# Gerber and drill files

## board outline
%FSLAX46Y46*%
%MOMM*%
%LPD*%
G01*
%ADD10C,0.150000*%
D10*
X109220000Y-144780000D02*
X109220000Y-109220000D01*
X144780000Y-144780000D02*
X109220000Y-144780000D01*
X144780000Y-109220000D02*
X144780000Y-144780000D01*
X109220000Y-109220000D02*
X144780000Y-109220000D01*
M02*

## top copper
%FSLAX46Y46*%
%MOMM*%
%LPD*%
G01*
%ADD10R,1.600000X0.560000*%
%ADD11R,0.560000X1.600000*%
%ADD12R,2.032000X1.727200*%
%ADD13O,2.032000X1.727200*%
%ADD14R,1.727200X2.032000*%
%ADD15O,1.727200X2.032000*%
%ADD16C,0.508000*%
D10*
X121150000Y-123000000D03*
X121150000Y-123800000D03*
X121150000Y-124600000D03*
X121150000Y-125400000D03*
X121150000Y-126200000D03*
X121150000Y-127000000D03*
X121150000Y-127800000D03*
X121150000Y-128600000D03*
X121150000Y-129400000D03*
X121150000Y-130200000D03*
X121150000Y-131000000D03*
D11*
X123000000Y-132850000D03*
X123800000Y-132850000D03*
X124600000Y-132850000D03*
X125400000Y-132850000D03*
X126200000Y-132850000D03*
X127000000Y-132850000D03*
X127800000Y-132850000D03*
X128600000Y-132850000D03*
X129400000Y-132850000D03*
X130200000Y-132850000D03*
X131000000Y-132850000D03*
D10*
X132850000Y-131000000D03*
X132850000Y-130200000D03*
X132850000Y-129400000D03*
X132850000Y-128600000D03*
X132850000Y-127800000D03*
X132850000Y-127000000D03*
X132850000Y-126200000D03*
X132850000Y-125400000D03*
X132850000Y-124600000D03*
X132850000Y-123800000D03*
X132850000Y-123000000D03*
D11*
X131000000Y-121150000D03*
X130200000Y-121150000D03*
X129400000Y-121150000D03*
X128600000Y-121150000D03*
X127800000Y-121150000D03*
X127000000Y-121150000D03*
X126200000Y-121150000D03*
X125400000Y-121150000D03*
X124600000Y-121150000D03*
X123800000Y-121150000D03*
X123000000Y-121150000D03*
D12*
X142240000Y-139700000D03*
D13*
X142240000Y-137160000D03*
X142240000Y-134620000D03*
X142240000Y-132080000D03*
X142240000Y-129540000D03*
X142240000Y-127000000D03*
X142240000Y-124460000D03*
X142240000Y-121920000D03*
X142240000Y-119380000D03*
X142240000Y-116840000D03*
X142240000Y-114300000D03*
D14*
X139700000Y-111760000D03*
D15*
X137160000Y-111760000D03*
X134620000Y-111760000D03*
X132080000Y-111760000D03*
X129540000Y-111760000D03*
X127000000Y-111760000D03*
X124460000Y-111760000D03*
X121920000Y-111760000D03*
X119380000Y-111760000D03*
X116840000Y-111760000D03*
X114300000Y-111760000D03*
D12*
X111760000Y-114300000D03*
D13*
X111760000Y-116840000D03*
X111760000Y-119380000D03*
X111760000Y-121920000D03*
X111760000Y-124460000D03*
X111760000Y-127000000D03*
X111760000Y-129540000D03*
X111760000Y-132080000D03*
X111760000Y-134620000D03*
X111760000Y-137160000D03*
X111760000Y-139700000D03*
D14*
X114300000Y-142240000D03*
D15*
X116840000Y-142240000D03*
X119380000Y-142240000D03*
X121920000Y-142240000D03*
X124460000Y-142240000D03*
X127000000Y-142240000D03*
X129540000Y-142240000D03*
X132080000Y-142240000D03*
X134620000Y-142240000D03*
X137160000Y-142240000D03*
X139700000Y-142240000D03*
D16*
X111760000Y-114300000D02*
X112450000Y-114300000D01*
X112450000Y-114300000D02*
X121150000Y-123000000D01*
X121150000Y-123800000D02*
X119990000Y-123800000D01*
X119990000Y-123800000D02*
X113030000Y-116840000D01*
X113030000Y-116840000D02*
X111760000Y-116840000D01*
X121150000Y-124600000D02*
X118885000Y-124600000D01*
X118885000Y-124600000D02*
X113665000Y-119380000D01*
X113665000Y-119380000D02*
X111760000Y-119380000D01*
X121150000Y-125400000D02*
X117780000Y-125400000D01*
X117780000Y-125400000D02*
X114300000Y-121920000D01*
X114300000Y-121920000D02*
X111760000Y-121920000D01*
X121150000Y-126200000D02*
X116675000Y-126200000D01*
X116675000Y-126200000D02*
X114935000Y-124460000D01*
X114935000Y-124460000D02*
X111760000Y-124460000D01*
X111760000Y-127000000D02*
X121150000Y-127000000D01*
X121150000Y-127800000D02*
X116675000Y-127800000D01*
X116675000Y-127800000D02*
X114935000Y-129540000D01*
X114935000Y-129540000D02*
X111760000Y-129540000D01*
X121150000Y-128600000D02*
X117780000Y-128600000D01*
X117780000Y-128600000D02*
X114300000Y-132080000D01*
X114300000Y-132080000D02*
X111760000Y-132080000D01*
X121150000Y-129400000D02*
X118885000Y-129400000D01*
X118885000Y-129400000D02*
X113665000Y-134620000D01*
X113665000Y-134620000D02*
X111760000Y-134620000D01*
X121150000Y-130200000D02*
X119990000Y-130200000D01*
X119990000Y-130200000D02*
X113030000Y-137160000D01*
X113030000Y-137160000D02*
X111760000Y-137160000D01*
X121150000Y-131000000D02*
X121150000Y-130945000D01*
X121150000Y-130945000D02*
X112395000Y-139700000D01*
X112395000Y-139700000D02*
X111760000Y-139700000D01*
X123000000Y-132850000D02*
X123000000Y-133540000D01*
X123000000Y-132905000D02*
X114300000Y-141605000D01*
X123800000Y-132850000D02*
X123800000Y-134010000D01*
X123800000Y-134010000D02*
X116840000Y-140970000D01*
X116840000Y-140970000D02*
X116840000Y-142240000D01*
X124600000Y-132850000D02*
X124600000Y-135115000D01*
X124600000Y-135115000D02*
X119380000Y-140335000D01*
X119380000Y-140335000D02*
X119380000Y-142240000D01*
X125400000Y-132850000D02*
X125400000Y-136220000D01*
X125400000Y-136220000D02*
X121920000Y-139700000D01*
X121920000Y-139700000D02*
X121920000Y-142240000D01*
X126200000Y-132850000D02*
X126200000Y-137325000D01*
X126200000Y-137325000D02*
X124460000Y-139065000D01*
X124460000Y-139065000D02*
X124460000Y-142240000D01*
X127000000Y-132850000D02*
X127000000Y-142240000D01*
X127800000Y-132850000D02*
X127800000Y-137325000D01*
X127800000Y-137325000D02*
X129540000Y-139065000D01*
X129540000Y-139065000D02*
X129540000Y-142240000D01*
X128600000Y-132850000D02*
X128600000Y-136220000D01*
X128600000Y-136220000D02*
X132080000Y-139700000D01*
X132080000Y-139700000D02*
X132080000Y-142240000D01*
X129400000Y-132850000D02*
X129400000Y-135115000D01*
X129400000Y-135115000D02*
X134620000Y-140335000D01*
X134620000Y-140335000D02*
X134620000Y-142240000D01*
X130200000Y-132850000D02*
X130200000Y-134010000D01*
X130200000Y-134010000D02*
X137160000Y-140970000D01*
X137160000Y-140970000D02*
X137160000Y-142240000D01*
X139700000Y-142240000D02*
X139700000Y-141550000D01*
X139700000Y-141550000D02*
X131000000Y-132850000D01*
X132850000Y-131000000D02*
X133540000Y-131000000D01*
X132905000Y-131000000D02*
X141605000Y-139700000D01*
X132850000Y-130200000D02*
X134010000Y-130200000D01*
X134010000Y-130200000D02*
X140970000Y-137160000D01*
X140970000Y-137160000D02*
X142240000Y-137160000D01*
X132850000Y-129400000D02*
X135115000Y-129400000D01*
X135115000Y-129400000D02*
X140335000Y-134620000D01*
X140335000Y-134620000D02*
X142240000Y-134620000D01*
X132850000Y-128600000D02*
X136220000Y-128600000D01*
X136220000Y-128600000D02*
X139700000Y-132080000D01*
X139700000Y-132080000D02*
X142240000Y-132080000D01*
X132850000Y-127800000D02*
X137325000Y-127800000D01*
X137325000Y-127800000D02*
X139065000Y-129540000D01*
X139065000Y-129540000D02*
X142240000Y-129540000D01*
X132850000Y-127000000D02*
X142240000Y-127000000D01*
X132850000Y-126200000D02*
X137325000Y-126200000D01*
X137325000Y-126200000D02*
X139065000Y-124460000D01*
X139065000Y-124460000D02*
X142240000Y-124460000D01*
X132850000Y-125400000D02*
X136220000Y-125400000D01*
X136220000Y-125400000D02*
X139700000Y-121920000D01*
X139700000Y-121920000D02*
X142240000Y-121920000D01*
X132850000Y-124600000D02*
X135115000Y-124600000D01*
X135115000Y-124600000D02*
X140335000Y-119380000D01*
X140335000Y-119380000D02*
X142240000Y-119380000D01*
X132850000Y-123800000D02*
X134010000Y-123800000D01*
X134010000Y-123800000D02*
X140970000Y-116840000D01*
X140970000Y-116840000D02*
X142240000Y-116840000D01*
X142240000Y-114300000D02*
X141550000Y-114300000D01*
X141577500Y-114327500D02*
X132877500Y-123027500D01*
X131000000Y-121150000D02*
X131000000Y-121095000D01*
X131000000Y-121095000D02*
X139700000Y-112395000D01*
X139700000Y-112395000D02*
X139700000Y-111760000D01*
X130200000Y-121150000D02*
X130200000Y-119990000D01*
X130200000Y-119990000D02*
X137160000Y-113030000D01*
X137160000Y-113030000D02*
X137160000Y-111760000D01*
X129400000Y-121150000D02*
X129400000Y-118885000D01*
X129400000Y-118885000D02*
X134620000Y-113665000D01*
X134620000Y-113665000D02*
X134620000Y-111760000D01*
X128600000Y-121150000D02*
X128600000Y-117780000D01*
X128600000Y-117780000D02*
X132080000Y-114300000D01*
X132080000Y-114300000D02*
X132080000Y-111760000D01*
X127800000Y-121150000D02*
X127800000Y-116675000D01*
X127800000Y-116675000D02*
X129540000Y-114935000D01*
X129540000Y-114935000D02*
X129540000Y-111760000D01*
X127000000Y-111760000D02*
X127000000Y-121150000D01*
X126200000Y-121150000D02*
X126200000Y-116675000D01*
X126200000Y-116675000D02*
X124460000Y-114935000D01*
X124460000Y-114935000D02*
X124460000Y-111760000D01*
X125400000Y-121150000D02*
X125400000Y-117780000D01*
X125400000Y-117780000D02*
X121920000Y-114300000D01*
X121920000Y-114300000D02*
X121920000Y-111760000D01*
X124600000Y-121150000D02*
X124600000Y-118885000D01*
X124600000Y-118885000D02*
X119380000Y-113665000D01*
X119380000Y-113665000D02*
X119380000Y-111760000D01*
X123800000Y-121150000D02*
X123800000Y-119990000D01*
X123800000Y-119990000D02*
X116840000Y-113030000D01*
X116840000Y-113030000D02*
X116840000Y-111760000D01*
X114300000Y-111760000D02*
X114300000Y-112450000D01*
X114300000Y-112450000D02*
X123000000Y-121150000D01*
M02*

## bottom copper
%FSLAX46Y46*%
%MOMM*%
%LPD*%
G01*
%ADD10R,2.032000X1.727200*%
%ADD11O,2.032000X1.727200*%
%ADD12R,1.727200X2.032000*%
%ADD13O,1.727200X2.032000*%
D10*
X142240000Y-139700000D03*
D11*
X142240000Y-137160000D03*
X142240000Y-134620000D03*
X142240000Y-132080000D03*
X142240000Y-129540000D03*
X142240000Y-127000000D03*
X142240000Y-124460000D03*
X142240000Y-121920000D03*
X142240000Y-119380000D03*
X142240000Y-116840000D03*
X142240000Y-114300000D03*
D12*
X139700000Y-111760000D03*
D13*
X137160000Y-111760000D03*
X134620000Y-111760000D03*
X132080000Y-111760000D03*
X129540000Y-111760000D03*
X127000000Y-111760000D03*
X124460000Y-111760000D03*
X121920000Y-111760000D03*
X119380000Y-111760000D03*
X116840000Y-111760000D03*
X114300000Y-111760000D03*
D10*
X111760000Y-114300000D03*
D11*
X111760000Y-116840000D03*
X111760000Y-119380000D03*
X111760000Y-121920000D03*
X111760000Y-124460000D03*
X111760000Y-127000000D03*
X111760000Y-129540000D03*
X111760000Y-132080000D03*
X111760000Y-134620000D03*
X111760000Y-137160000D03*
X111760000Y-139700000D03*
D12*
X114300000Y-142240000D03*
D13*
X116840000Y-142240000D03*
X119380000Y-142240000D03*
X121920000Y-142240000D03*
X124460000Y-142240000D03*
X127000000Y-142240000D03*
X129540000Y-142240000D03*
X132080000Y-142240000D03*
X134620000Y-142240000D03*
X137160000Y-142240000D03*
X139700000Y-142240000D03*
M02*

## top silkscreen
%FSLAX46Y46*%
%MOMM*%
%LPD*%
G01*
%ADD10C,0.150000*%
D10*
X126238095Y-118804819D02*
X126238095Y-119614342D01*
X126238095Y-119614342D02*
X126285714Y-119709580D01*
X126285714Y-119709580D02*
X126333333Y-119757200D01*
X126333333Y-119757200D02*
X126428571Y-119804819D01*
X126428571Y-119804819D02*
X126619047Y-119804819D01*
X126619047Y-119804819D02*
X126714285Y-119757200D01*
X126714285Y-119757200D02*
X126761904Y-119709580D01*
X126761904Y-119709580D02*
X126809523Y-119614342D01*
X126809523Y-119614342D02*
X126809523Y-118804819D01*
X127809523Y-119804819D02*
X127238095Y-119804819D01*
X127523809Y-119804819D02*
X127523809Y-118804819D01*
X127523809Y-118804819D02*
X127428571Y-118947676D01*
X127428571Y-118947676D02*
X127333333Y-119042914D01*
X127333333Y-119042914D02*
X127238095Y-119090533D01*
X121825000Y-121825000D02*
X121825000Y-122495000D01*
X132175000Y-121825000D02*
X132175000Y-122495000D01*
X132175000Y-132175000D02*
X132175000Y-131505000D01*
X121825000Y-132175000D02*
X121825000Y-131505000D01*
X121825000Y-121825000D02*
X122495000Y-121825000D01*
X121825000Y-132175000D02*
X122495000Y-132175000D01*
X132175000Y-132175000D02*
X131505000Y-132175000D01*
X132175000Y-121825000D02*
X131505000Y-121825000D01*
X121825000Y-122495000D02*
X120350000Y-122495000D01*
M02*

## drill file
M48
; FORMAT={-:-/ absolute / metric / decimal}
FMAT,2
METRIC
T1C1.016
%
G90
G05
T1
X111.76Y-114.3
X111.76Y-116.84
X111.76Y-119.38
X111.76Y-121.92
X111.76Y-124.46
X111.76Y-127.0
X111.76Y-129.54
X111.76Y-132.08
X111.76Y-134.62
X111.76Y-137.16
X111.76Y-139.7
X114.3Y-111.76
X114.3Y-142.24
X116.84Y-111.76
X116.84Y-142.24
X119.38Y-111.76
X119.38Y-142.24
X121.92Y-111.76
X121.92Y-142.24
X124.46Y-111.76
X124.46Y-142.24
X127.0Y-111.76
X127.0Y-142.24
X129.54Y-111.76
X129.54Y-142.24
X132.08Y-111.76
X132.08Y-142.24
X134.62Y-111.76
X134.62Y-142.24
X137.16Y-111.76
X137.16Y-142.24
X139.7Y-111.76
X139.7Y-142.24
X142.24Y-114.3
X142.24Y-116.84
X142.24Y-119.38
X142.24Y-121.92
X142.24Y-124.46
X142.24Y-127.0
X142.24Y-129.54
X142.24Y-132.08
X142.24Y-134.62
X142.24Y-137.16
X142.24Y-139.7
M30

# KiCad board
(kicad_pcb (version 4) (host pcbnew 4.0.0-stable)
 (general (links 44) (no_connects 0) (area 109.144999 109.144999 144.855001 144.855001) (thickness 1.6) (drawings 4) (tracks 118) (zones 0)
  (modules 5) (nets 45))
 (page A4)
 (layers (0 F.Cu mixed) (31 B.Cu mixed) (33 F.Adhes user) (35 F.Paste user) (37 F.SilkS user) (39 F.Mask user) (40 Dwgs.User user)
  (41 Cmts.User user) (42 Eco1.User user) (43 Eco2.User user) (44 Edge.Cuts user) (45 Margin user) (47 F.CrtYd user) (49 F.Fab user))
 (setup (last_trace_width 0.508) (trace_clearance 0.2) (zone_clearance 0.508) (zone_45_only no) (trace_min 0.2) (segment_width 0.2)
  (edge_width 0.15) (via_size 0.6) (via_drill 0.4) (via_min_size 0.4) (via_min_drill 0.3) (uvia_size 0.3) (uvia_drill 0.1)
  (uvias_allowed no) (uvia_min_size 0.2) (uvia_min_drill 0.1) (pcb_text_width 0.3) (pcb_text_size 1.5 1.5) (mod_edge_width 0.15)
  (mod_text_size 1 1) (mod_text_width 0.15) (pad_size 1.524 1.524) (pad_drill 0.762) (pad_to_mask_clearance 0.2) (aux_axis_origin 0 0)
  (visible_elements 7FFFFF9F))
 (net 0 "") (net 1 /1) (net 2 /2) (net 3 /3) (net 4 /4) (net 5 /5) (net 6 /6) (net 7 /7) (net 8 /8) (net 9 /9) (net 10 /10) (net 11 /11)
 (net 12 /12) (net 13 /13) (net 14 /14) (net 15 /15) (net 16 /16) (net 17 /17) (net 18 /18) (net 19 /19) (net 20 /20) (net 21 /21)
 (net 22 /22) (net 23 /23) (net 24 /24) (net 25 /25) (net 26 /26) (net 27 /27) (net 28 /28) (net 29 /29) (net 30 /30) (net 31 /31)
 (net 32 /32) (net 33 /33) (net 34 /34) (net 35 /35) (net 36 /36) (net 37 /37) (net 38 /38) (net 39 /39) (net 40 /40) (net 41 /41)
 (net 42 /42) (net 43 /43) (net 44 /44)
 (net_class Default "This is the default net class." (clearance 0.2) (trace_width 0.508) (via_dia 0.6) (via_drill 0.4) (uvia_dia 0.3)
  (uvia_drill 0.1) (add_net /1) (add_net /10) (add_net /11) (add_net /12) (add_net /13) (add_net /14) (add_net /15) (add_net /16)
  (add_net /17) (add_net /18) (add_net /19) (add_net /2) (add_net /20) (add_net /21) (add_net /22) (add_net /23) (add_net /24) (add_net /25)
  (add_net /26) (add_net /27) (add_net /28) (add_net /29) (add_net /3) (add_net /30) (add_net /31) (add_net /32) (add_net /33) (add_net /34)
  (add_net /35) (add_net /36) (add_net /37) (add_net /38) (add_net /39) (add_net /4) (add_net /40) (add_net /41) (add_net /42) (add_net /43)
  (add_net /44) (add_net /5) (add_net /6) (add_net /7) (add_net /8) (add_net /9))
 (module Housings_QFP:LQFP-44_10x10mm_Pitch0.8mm (layer F.Cu) (at 127 127)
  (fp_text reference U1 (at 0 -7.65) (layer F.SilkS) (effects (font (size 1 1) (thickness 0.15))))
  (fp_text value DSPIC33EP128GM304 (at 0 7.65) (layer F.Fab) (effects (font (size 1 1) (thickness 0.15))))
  (fp_line (start -5.175 -5.175) (end -5.175 -4.505) (layer F.SilkS) (width 0.15))
  (fp_line (start 5.175 -5.175) (end 5.175 -4.505) (layer F.SilkS) (width 0.15))
  (fp_line (start 5.175 5.175) (end 5.175 4.505) (layer F.SilkS) (width 0.15))
  (fp_line (start -5.175 5.175) (end -5.175 4.505) (layer F.SilkS) (width 0.15))
  (fp_line (start -5.175 -5.175) (end -4.505 -5.175) (layer F.SilkS) (width 0.15))
  (fp_line (start -5.175 5.175) (end -4.505 5.175) (layer F.SilkS) (width 0.15))
  (fp_line (start 5.175 5.175) (end 4.505 5.175) (layer F.SilkS) (width 0.15))
  (fp_line (start 5.175 -5.175) (end 4.505 -5.175) (layer F.SilkS) (width 0.15))
  (fp_line (start -5.175 -4.505) (end -6.65 -4.505) (layer F.SilkS) (width 0.15))
  (pad 1 smd rect (at -5.85 -4) (size 1.6 0.56) (layers F.Cu F.Paste F.Mask) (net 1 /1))
  (pad 2 smd rect (at -5.85 -3.2) (size 1.6 0.56) (layers F.Cu F.Paste F.Mask) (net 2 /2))
  (pad 3 smd rect (at -5.85 -2.4) (size 1.6 0.56) (layers F.Cu F.Paste F.Mask) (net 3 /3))
  (pad 4 smd rect (at -5.85 -1.6) (size 1.6 0.56) (layers F.Cu F.Paste F.Mask) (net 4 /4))
  (pad 5 smd rect (at -5.85 -0.8) (size 1.6 0.56) (layers F.Cu F.Paste F.Mask) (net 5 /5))
  (pad 6 smd rect (at -5.85 0) (size 1.6 0.56) (layers F.Cu F.Paste F.Mask) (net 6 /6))
  (pad 7 smd rect (at -5.85 0.8) (size 1.6 0.56) (layers F.Cu F.Paste F.Mask) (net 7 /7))
  (pad 8 smd rect (at -5.85 1.6) (size 1.6 0.56) (layers F.Cu F.Paste F.Mask) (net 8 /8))
  (pad 9 smd rect (at -5.85 2.4) (size 1.6 0.56) (layers F.Cu F.Paste F.Mask) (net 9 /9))
  (pad 10 smd rect (at -5.85 3.2) (size 1.6 0.56) (layers F.Cu F.Paste F.Mask) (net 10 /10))
  (pad 11 smd rect (at -5.85 4) (size 1.6 0.56) (layers F.Cu F.Paste F.Mask) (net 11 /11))
  (pad 12 smd rect (at -4 5.85 90) (size 1.6 0.56) (layers F.Cu F.Paste F.Mask) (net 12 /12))
  (pad 13 smd rect (at -3.2 5.85 90) (size 1.6 0.56) (layers F.Cu F.Paste F.Mask) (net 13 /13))
  (pad 14 smd rect (at -2.4 5.85 90) (size 1.6 0.56) (layers F.Cu F.Paste F.Mask) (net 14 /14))
  (pad 15 smd rect (at -1.6 5.85 90) (size 1.6 0.56) (layers F.Cu F.Paste F.Mask) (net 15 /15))
  (pad 16 smd rect (at -0.8 5.85 90) (size 1.6 0.56) (layers F.Cu F.Paste F.Mask) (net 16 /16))
  (pad 17 smd rect (at 0 5.85 90) (size 1.6 0.56) (layers F.Cu F.Paste F.Mask) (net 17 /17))
  (pad 18 smd rect (at 0.8 5.85 90) (size 1.6 0.56) (layers F.Cu F.Paste F.Mask) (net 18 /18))
  (pad 19 smd rect (at 1.6 5.85 90) (size 1.6 0.56) (layers F.Cu F.Paste F.Mask) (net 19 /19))
  (pad 20 smd rect (at 2.4 5.85 90) (size 1.6 0.56) (layers F.Cu F.Paste F.Mask) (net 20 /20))
  (pad 21 smd rect (at 3.2 5.85 90) (size 1.6 0.56) (layers F.Cu F.Paste F.Mask) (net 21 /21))
  (pad 22 smd rect (at 4 5.85 90) (size 1.6 0.56) (layers F.Cu F.Paste F.Mask) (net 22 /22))
  (pad 23 smd rect (at 5.85 4) (size 1.6 0.56) (layers F.Cu F.Paste F.Mask) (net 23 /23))
  (pad 24 smd rect (at 5.85 3.2) (size 1.6 0.56) (layers F.Cu F.Paste F.Mask) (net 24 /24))
  (pad 25 smd rect (at 5.85 2.4) (size 1.6 0.56) (layers F.Cu F.Paste F.Mask) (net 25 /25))
  (pad 26 smd rect (at 5.85 1.6) (size 1.6 0.56) (layers F.Cu F.Paste F.Mask) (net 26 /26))
  (pad 27 smd rect (at 5.85 0.8) (size 1.6 0.56) (layers F.Cu F.Paste F.Mask) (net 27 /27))
  (pad 28 smd rect (at 5.85 0) (size 1.6 0.56) (layers F.Cu F.Paste F.Mask) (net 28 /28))
  (pad 29 smd rect (at 5.85 -0.8) (size 1.6 0.56) (layers F.Cu F.Paste F.Mask) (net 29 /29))
  (pad 30 smd rect (at 5.85 -1.6) (size 1.6 0.56) (layers F.Cu F.Paste F.Mask) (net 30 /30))
  (pad 31 smd rect (at 5.85 -2.4) (size 1.6 0.56) (layers F.Cu F.Paste F.Mask) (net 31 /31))
  (pad 32 smd rect (at 5.85 -3.2) (size 1.6 0.56) (layers F.Cu F.Paste F.Mask) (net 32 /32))
  (pad 33 smd rect (at 5.85 -4) (size 1.6 0.56) (layers F.Cu F.Paste F.Mask) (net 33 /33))
  (pad 34 smd rect (at 4 -5.85 90) (size 1.6 0.56) (layers F.Cu F.Paste F.Mask) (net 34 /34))
  (pad 35 smd rect (at 3.2 -5.85 90) (size 1.6 0.56) (layers F.Cu F.Paste F.Mask) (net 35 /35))
  (pad 36 smd rect (at 2.4 -5.85 90) (size 1.6 0.56) (layers F.Cu F.Paste F.Mask) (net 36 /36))
  (pad 37 smd rect (at 1.6 -5.85 90) (size 1.6 0.56) (layers F.Cu F.Paste F.Mask) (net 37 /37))
  (pad 38 smd rect (at 0.8 -5.85 90) (size 1.6 0.56) (layers F.Cu F.Paste F.Mask) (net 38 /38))
  (pad 39 smd rect (at 0 -5.85 90) (size 1.6 0.56) (layers F.Cu F.Paste F.Mask) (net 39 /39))
  (pad 40 smd rect (at -0.8 -5.85 90) (size 1.6 0.56) (layers F.Cu F.Paste F.Mask) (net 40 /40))
  (pad 41 smd rect (at -1.6 -5.85 90) (size 1.6 0.56) (layers F.Cu F.Paste F.Mask) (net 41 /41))
  (pad 42 smd rect (at -2.4 -5.85 90) (size 1.6 0.56) (layers F.Cu F.Paste F.Mask) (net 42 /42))
  (pad 43 smd rect (at -3.2 -5.85 90) (size 1.6 0.56) (layers F.Cu F.Paste F.Mask) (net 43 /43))
  (pad 44 smd rect (at -4 -5.85 90) (size 1.6 0.56) (layers F.Cu F.Paste F.Mask) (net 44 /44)))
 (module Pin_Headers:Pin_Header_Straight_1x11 (layer B.Cu) (at 142.24 139.7)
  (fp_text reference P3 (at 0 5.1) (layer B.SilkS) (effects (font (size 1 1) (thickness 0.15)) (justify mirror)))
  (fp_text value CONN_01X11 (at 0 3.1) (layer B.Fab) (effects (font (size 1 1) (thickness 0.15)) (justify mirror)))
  (pad 1 thru_hole rect (at 0 0) (size 2.032 1.7272) (drill 1.016) (layers *.Cu *.Mask) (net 23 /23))
  (pad 2 thru_hole oval (at 0 -2.54) (size 2.032 1.7272) (drill 1.016) (layers *.Cu *.Mask) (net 24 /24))
  (pad 3 thru_hole oval (at 0 -5.08) (size 2.032 1.7272) (drill 1.016) (layers *.Cu *.Mask) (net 25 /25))
  (pad 4 thru_hole oval (at 0 -7.62) (size 2.032 1.7272) (drill 1.016) (layers *.Cu *.Mask) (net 26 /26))
  (pad 5 thru_hole oval (at 0 -10.16) (size 2.032 1.7272) (drill 1.016) (layers *.Cu *.Mask) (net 27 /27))
  (pad 6 thru_hole oval (at 0 -12.7) (size 2.032 1.7272) (drill 1.016) (layers *.Cu *.Mask) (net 28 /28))
  (pad 7 thru_hole oval (at 0 -15.24) (size 2.032 1.7272) (drill 1.016) (layers *.Cu *.Mask) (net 29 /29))
  (pad 8 thru_hole oval (at 0 -17.78) (size 2.032 1.7272) (drill 1.016) (layers *.Cu *.Mask) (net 30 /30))
  (pad 9 thru_hole oval (at 0 -20.32) (size 2.032 1.7272) (drill 1.016) (layers *.Cu *.Mask) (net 31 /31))
  (pad 10 thru_hole oval (at 0 -22.86) (size 2.032 1.7272) (drill 1.016) (layers *.Cu *.Mask) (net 32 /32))
  (pad 11 thru_hole oval (at 0 -25.4) (size 2.032 1.7272) (drill 1.016) (layers *.Cu *.Mask) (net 33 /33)))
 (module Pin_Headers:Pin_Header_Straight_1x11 (layer B.Cu) (at 139.7 111.76 90)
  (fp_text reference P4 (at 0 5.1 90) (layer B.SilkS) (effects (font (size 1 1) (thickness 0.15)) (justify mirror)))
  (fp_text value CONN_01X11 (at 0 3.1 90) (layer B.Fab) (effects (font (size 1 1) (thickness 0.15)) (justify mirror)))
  (pad 1 thru_hole rect (at 0 0 90) (size 2.032 1.7272) (drill 1.016) (layers *.Cu *.Mask) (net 34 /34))
  (pad 2 thru_hole oval (at 0 -2.54 90) (size 2.032 1.7272) (drill 1.016) (layers *.Cu *.Mask) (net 35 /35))
  (pad 3 thru_hole oval (at 0 -5.08 90) (size 2.032 1.7272) (drill 1.016) (layers *.Cu *.Mask) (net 36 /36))
  (pad 4 thru_hole oval (at 0 -7.62 90) (size 2.032 1.7272) (drill 1.016) (layers *.Cu *.Mask) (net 37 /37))
  (pad 5 thru_hole oval (at 0 -10.16 90) (size 2.032 1.7272) (drill 1.016) (layers *.Cu *.Mask) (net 38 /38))
  (pad 6 thru_hole oval (at 0 -12.7 90) (size 2.032 1.7272) (drill 1.016) (layers *.Cu *.Mask) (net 39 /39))
  (pad 7 thru_hole oval (at 0 -15.24 90) (size 2.032 1.7272) (drill 1.016) (layers *.Cu *.Mask) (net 40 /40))
  (pad 8 thru_hole oval (at 0 -17.78 90) (size 2.032 1.7272) (drill 1.016) (layers *.Cu *.Mask) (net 41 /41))
  (pad 9 thru_hole oval (at 0 -20.32 90) (size 2.032 1.7272) (drill 1.016) (layers *.Cu *.Mask) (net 42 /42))
  (pad 10 thru_hole oval (at 0 -22.86 90) (size 2.032 1.7272) (drill 1.016) (layers *.Cu *.Mask) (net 43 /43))
  (pad 11 thru_hole oval (at 0 -25.4 90) (size 2.032 1.7272) (drill 1.016) (layers *.Cu *.Mask) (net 44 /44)))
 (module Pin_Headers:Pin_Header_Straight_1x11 (layer B.Cu) (at 111.76 114.3 180)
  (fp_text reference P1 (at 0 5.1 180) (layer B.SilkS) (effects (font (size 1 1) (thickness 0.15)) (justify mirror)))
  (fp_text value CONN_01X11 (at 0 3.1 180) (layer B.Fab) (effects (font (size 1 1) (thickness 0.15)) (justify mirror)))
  (pad 1 thru_hole rect (at 0 0 180) (size 2.032 1.7272) (drill 1.016) (layers *.Cu *.Mask) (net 1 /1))
  (pad 2 thru_hole oval (at 0 -2.54 180) (size 2.032 1.7272) (drill 1.016) (layers *.Cu *.Mask) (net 2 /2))
  (pad 3 thru_hole oval (at 0 -5.08 180) (size 2.032 1.7272) (drill 1.016) (layers *.Cu *.Mask) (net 3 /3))
  (pad 4 thru_hole oval (at 0 -7.62 180) (size 2.032 1.7272) (drill 1.016) (layers *.Cu *.Mask) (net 4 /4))
  (pad 5 thru_hole oval (at 0 -10.16 180) (size 2.032 1.7272) (drill 1.016) (layers *.Cu *.Mask) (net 5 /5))
  (pad 6 thru_hole oval (at 0 -12.7 180) (size 2.032 1.7272) (drill 1.016) (layers *.Cu *.Mask) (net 6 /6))
  (pad 7 thru_hole oval (at 0 -15.24 180) (size 2.032 1.7272) (drill 1.016) (layers *.Cu *.Mask) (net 7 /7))
  (pad 8 thru_hole oval (at 0 -17.78 180) (size 2.032 1.7272) (drill 1.016) (layers *.Cu *.Mask) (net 8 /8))
  (pad 9 thru_hole oval (at 0 -20.32 180) (size 2.032 1.7272) (drill 1.016) (layers *.Cu *.Mask) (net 9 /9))
  (pad 10 thru_hole oval (at 0 -22.86 180) (size 2.032 1.7272) (drill 1.016) (layers *.Cu *.Mask) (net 10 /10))
  (pad 11 thru_hole oval (at 0 -25.4 180) (size 2.032 1.7272) (drill 1.016) (layers *.Cu *.Mask) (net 11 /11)))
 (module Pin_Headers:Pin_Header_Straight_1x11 (layer B.Cu) (at 114.3 142.24 270)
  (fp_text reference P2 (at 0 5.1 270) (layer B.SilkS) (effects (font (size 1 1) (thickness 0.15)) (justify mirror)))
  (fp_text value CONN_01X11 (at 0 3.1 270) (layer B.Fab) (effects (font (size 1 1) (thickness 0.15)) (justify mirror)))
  (pad 1 thru_hole rect (at 0 0 270) (size 2.032 1.7272) (drill 1.016) (layers *.Cu *.Mask) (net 12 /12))
  (pad 2 thru_hole oval (at 0 -2.54 270) (size 2.032 1.7272) (drill 1.016) (layers *.Cu *.Mask) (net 13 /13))
  (pad 3 thru_hole oval (at 0 -5.08 270) (size 2.032 1.7272) (drill 1.016) (layers *.Cu *.Mask) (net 14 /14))
  (pad 4 thru_hole oval (at 0 -7.62 270) (size 2.032 1.7272) (drill 1.016) (layers *.Cu *.Mask) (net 15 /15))
  (pad 5 thru_hole oval (at 0 -10.16 270) (size 2.032 1.7272) (drill 1.016) (layers *.Cu *.Mask) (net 16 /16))
  (pad 6 thru_hole oval (at 0 -12.7 270) (size 2.032 1.7272) (drill 1.016) (layers *.Cu *.Mask) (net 17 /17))
  (pad 7 thru_hole oval (at 0 -15.24 270) (size 2.032 1.7272) (drill 1.016) (layers *.Cu *.Mask) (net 18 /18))
  (pad 8 thru_hole oval (at 0 -17.78 270) (size 2.032 1.7272) (drill 1.016) (layers *.Cu *.Mask) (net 19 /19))
  (pad 9 thru_hole oval (at 0 -20.32 270) (size 2.032 1.7272) (drill 1.016) (layers *.Cu *.Mask) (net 20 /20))
  (pad 10 thru_hole oval (at 0 -22.86 270) (size 2.032 1.7272) (drill 1.016) (layers *.Cu *.Mask) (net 21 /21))
  (pad 11 thru_hole oval (at 0 -25.4 270) (size 2.032 1.7272) (drill 1.016) (layers *.Cu *.Mask) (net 22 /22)))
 (gr_line (start 109.22 144.78) (end 109.22 109.22) (angle 90) (layer Edge.Cuts) (width 0.15))
 (gr_line (start 144.78 144.78) (end 109.22 144.78) (angle 90) (layer Edge.Cuts) (width 0.15))
 (gr_line (start 144.78 109.22) (end 144.78 144.78) (angle 90) (layer Edge.Cuts) (width 0.15))
 (gr_line (start 109.22 109.22) (end 144.78 109.22) (angle 90) (layer Edge.Cuts) (width 0.15))
 (segment (start 111.76 114.3) (end 112.45 114.3) (width 0.508) (layer F.Cu) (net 1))
 (segment (start 112.45 114.3) (end 121.15 123) (width 0.508) (layer F.Cu) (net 1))
 (segment (start 121.15 123.8) (end 119.99 123.8) (width 0.508) (layer F.Cu) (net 2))
 (segment (start 119.99 123.8) (end 113.03 116.84) (width 0.508) (layer F.Cu) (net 2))
 (segment (start 113.03 116.84) (end 111.76 116.84) (width 0.508) (layer F.Cu) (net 2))
 (segment (start 121.15 124.6) (end 118.885 124.6) (width 0.508) (layer F.Cu) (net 3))
 (segment (start 118.885 124.6) (end 113.665 119.38) (width 0.508) (layer F.Cu) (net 3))
 (segment (start 113.665 119.38) (end 111.76 119.38) (width 0.508) (layer F.Cu) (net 3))
 (segment (start 121.15 125.4) (end 117.78 125.4) (width 0.508) (layer F.Cu) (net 4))
 (segment (start 117.78 125.4) (end 114.3 121.92) (width 0.508) (layer F.Cu) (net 4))
 (segment (start 114.3 121.92) (end 111.76 121.92) (width 0.508) (layer F.Cu) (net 4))
 (segment (start 121.15 126.2) (end 116.675 126.2) (width 0.508) (layer F.Cu) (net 5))
 (segment (start 116.675 126.2) (end 114.935 124.46) (width 0.508) (layer F.Cu) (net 5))
 (segment (start 114.935 124.46) (end 111.76 124.46) (width 0.508) (layer F.Cu) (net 5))
 (segment (start 111.76 127) (end 121.15 127) (width 0.508) (layer F.Cu) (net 6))
 (segment (start 121.15 127.8) (end 116.675 127.8) (width 0.508) (layer F.Cu) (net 7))
 (segment (start 116.675 127.8) (end 114.935 129.54) (width 0.508) (layer F.Cu) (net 7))
 (segment (start 114.935 129.54) (end 111.76 129.54) (width 0.508) (layer F.Cu) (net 7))
 (segment (start 121.15 128.6) (end 117.78 128.6) (width 0.508) (layer F.Cu) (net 8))
 (segment (start 117.78 128.6) (end 114.3 132.08) (width 0.508) (layer F.Cu) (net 8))
 (segment (start 114.3 132.08) (end 111.76 132.08) (width 0.508) (layer F.Cu) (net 8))
 (segment (start 121.15 129.4) (end 118.885 129.4) (width 0.508) (layer F.Cu) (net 9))
 (segment (start 118.885 129.4) (end 113.665 134.62) (width 0.508) (layer F.Cu) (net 9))
 (segment (start 113.665 134.62) (end 111.76 134.62) (width 0.508) (layer F.Cu) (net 9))
 (segment (start 121.15 130.2) (end 119.99 130.2) (width 0.508) (layer F.Cu) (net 10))
 (segment (start 119.99 130.2) (end 113.03 137.16) (width 0.508) (layer F.Cu) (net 10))
 (segment (start 113.03 137.16) (end 111.76 137.16) (width 0.508) (layer F.Cu) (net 10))
 (segment (start 121.15 131) (end 121.15 130.945) (width 0.508) (layer F.Cu) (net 11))
 (segment (start 121.15 130.945) (end 112.395 139.7) (width 0.508) (layer F.Cu) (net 11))
 (segment (start 112.395 139.7) (end 111.76 139.7) (width 0.508) (layer F.Cu) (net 11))
 (segment (start 123 132.85) (end 123 133.54) (width 0.508) (layer F.Cu) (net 12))
 (segment (start 123 132.905) (end 114.3 141.605) (width 0.508) (layer F.Cu) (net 12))
 (segment (start 123.8 132.85) (end 123.8 134.01) (width 0.508) (layer F.Cu) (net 13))
 (segment (start 123.8 134.01) (end 116.84 140.97) (width 0.508) (layer F.Cu) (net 13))
 (segment (start 116.84 140.97) (end 116.84 142.24) (width 0.508) (layer F.Cu) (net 13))
 (segment (start 124.6 132.85) (end 124.6 135.115) (width 0.508) (layer F.Cu) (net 14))
 (segment (start 124.6 135.115) (end 119.38 140.335) (width 0.508) (layer F.Cu) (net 14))
 (segment (start 119.38 140.335) (end 119.38 142.24) (width 0.508) (layer F.Cu) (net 14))
 (segment (start 125.4 132.85) (end 125.4 136.22) (width 0.508) (layer F.Cu) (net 15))
 (segment (start 125.4 136.22) (end 121.92 139.7) (width 0.508) (layer F.Cu) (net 15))
 (segment (start 121.92 139.7) (end 121.92 142.24) (width 0.508) (layer F.Cu) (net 15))
 (segment (start 126.2 132.85) (end 126.2 137.325) (width 0.508) (layer F.Cu) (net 16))
 (segment (start 126.2 137.325) (end 124.46 139.065) (width 0.508) (layer F.Cu) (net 16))
 (segment (start 124.46 139.065) (end 124.46 142.24) (width 0.508) (layer F.Cu) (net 16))
 (segment (start 127 132.85) (end 127 142.24) (width 0.508) (layer F.Cu) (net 17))
 (segment (start 127.8 132.85) (end 127.8 137.325) (width 0.508) (layer F.Cu) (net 18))
 (segment (start 127.8 137.325) (end 129.54 139.065) (width 0.508) (layer F.Cu) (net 18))
 (segment (start 129.54 139.065) (end 129.54 142.24) (width 0.508) (layer F.Cu) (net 18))
 (segment (start 128.6 132.85) (end 128.6 136.22) (width 0.508) (layer F.Cu) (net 19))
 (segment (start 128.6 136.22) (end 132.08 139.7) (width 0.508) (layer F.Cu) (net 19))
 (segment (start 132.08 139.7) (end 132.08 142.24) (width 0.508) (layer F.Cu) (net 19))
 (segment (start 129.4 132.85) (end 129.4 135.115) (width 0.508) (layer F.Cu) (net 20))
 (segment (start 129.4 135.115) (end 134.62 140.335) (width 0.508) (layer F.Cu) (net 20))
 (segment (start 134.62 140.335) (end 134.62 142.24) (width 0.508) (layer F.Cu) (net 20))
 (segment (start 130.2 132.85) (end 130.2 134.01) (width 0.508) (layer F.Cu) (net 21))
 (segment (start 130.2 134.01) (end 137.16 140.97) (width 0.508) (layer F.Cu) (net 21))
 (segment (start 137.16 140.97) (end 137.16 142.24) (width 0.508) (layer F.Cu) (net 21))
 (segment (start 139.7 142.24) (end 139.7 141.55) (width 0.508) (layer F.Cu) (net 22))
 (segment (start 139.7 141.55) (end 131 132.85) (width 0.508) (layer F.Cu) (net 22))
 (segment (start 132.85 131) (end 133.54 131) (width 0.508) (layer F.Cu) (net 23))
 (segment (start 132.905 131) (end 141.605 139.7) (width 0.508) (layer F.Cu) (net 23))
 (segment (start 132.85 130.2) (end 134.01 130.2) (width 0.508) (layer F.Cu) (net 24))
 (segment (start 134.01 130.2) (end 140.97 137.16) (width 0.508) (layer F.Cu) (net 24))
 (segment (start 140.97 137.16) (end 142.24 137.16) (width 0.508) (layer F.Cu) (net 24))
 (segment (start 132.85 129.4) (end 135.115 129.4) (width 0.508) (layer F.Cu) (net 25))
 (segment (start 135.115 129.4) (end 140.335 134.62) (width 0.508) (layer F.Cu) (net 25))
 (segment (start 140.335 134.62) (end 142.24 134.62) (width 0.508) (layer F.Cu) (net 25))
 (segment (start 132.85 128.6) (end 136.22 128.6) (width 0.508) (layer F.Cu) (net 26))
 (segment (start 136.22 128.6) (end 139.7 132.08) (width 0.508) (layer F.Cu) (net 26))
 (segment (start 139.7 132.08) (end 142.24 132.08) (width 0.508) (layer F.Cu) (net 26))
 (segment (start 132.85 127.8) (end 137.325 127.8) (width 0.508) (layer F.Cu) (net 27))
 (segment (start 137.325 127.8) (end 139.065 129.54) (width 0.508) (layer F.Cu) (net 27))
 (segment (start 139.065 129.54) (end 142.24 129.54) (width 0.508) (layer F.Cu) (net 27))
 (segment (start 132.85 127) (end 142.24 127) (width 0.508) (layer F.Cu) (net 28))
 (segment (start 132.85 126.2) (end 137.325 126.2) (width 0.508) (layer F.Cu) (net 29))
 (segment (start 137.325 126.2) (end 139.065 124.46) (width 0.508) (layer F.Cu) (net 29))
 (segment (start 139.065 124.46) (end 142.24 124.46) (width 0.508) (layer F.Cu) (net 29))
 (segment (start 132.85 125.4) (end 136.22 125.4) (width 0.508) (layer F.Cu) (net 30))
 (segment (start 136.22 125.4) (end 139.7 121.92) (width 0.508) (layer F.Cu) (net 30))
 (segment (start 139.7 121.92) (end 142.24 121.92) (width 0.508) (layer F.Cu) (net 30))
 (segment (start 132.85 124.6) (end 135.115 124.6) (width 0.508) (layer F.Cu) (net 31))
 (segment (start 135.115 124.6) (end 140.335 119.38) (width 0.508) (layer F.Cu) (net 31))
 (segment (start 140.335 119.38) (end 142.24 119.38) (width 0.508) (layer F.Cu) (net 31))
 (segment (start 132.85 123.8) (end 134.01 123.8) (width 0.508) (layer F.Cu) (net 32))
 (segment (start 134.01 123.8) (end 140.97 116.84) (width 0.508) (layer F.Cu) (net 32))
 (segment (start 140.97 116.84) (end 142.24 116.84) (width 0.508) (layer F.Cu) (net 32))
 (segment (start 142.24 114.3) (end 141.55 114.3) (width 0.508) (layer F.Cu) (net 33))
 (segment (start 141.5775 114.3275) (end 132.8775 123.0275) (width 0.508) (layer F.Cu) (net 33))
 (segment (start 131 121.15) (end 131 121.095) (width 0.508) (layer F.Cu) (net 34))
 (segment (start 131 121.095) (end 139.7 112.395) (width 0.508) (layer F.Cu) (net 34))
 (segment (start 139.7 112.395) (end 139.7 111.76) (width 0.508) (layer F.Cu) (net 34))
 (segment (start 130.2 121.15) (end 130.2 119.99) (width 0.508) (layer F.Cu) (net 35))
 (segment (start 130.2 119.99) (end 137.16 113.03) (width 0.508) (layer F.Cu) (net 35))
 (segment (start 137.16 113.03) (end 137.16 111.76) (width 0.508) (layer F.Cu) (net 35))
 (segment (start 129.4 121.15) (end 129.4 118.885) (width 0.508) (layer F.Cu) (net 36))
 (segment (start 129.4 118.885) (end 134.62 113.665) (width 0.508) (layer F.Cu) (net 36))
 (segment (start 134.62 113.665) (end 134.62 111.76) (width 0.508) (layer F.Cu) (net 36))
 (segment (start 128.6 121.15) (end 128.6 117.78) (width 0.508) (layer F.Cu) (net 37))
 (segment (start 128.6 117.78) (end 132.08 114.3) (width 0.508) (layer F.Cu) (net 37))
 (segment (start 132.08 114.3) (end 132.08 111.76) (width 0.508) (layer F.Cu) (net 37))
 (segment (start 127.8 121.15) (end 127.8 116.675) (width 0.508) (layer F.Cu) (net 38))
 (segment (start 127.8 116.675) (end 129.54 114.935) (width 0.508) (layer F.Cu) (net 38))
 (segment (start 129.54 114.935) (end 129.54 111.76) (width 0.508) (layer F.Cu) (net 38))
 (segment (start 127 111.76) (end 127 121.15) (width 0.508) (layer F.Cu) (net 39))
 (segment (start 126.2 121.15) (end 126.2 116.675) (width 0.508) (layer F.Cu) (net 40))
 (segment (start 126.2 116.675) (end 124.46 114.935) (width 0.508) (layer F.Cu) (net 40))
 (segment (start 124.46 114.935) (end 124.46 111.76) (width 0.508) (layer F.Cu) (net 40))
 (segment (start 125.4 121.15) (end 125.4 117.78) (width 0.508) (layer F.Cu) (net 41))
 (segment (start 125.4 117.78) (end 121.92 114.3) (width 0.508) (layer F.Cu) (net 41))
 (segment (start 121.92 114.3) (end 121.92 111.76) (width 0.508) (layer F.Cu) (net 41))
 (segment (start 124.6 121.15) (end 124.6 118.885) (width 0.508) (layer F.Cu) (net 42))
 (segment (start 124.6 118.885) (end 119.38 113.665) (width 0.508) (layer F.Cu) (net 42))
 (segment (start 119.38 113.665) (end 119.38 111.76) (width 0.508) (layer F.Cu) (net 42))
 (segment (start 123.8 121.15) (end 123.8 119.99) (width 0.508) (layer F.Cu) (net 43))
 (segment (start 123.8 119.99) (end 116.84 113.03) (width 0.508) (layer F.Cu) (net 43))
 (segment (start 116.84 113.03) (end 116.84 111.76) (width 0.508) (layer F.Cu) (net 43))
 (segment (start 114.3 111.76) (end 114.3 112.45) (width 0.508) (layer F.Cu) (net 44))
 (segment (start 114.3 112.45) (end 123 121.15) (width 0.508) (layer F.Cu) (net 44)))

